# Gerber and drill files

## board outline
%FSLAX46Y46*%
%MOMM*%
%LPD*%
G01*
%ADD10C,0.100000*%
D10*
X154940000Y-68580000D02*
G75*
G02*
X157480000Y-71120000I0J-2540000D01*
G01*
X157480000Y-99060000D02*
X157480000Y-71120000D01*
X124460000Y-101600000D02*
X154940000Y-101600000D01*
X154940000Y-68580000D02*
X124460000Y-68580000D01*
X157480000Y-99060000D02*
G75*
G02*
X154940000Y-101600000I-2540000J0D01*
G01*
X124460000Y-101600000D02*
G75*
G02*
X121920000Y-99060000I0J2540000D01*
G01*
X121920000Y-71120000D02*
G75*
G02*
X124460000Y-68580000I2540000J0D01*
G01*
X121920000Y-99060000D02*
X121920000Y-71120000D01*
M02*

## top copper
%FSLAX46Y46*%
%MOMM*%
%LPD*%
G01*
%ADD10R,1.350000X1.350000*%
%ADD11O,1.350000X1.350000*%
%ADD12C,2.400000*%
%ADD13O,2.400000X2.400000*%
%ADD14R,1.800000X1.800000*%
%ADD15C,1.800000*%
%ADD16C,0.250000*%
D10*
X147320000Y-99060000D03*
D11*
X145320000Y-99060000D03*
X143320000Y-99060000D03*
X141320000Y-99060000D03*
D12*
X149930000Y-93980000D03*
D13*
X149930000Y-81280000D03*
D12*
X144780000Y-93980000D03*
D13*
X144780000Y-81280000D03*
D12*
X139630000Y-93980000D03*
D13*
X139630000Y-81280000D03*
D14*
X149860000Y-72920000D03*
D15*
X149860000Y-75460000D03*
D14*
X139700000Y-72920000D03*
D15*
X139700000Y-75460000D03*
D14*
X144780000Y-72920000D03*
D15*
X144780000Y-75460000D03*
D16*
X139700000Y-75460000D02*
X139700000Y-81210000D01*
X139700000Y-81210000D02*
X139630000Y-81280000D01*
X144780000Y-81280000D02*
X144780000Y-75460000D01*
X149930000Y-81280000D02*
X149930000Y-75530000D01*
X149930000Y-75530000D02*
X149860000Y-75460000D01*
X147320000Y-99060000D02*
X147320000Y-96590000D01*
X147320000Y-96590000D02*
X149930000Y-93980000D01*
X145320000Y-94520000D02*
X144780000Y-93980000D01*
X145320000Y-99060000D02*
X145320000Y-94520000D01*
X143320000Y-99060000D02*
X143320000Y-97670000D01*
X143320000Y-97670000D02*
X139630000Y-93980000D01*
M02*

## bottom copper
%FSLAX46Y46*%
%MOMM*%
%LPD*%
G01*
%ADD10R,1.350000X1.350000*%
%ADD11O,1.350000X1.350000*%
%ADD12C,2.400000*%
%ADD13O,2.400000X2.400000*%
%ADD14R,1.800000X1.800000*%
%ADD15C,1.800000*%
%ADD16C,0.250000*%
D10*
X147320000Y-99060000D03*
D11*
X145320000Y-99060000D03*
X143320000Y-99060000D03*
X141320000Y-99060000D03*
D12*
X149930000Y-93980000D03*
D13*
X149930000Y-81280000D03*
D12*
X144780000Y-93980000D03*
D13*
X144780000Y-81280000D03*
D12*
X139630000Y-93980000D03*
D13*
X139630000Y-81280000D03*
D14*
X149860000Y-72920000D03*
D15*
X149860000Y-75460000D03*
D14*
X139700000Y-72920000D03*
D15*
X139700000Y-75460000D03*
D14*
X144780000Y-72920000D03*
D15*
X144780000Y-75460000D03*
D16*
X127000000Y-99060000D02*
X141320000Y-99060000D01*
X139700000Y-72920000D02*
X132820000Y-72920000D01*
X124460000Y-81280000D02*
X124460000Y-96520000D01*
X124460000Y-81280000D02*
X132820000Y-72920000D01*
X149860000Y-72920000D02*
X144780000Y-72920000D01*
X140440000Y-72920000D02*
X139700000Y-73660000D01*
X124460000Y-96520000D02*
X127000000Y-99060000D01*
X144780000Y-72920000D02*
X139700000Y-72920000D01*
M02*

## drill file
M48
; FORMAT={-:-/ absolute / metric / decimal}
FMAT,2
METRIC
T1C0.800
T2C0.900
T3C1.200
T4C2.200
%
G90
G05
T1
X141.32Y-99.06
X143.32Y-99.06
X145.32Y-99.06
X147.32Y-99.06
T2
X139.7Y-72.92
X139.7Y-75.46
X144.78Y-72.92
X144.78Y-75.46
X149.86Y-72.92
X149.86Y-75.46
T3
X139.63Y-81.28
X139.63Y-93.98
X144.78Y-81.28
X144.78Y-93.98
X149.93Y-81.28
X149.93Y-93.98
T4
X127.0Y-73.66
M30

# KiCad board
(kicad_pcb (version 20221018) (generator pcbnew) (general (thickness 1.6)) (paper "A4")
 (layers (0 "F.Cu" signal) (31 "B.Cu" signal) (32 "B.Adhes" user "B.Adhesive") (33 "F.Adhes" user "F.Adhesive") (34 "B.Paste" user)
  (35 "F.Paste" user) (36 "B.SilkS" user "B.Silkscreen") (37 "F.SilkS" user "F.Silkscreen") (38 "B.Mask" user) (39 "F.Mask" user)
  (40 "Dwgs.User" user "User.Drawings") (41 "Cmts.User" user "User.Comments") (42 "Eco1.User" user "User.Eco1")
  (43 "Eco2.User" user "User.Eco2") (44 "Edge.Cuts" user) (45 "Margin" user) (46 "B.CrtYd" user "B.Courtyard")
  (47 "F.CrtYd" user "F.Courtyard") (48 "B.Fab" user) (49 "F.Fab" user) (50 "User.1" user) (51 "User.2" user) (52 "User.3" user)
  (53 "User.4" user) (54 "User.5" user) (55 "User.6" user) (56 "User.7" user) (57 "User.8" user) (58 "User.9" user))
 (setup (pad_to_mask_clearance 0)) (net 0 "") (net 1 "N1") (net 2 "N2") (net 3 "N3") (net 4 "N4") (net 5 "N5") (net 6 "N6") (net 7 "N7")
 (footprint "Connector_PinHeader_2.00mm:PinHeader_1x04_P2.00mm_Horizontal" (layer "F.Cu") (at 147.32 99.06 -90)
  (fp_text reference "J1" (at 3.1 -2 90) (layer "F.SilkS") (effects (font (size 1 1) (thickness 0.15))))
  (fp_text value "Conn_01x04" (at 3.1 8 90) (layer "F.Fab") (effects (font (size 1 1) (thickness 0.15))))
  (pad "1" thru_hole rect (at 0 0 270) (size 1.35 1.35) (drill 0.8) (layers "*.Cu" "*.Mask") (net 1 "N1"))
  (pad "2" thru_hole oval (at 0 2 270) (size 1.35 1.35) (drill 0.8) (layers "*.Cu" "*.Mask") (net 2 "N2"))
  (pad "3" thru_hole oval (at 0 4 270) (size 1.35 1.35) (drill 0.8) (layers "*.Cu" "*.Mask") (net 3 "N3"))
  (pad "4" thru_hole oval (at 0 6 270) (size 1.35 1.35) (drill 0.8) (layers "*.Cu" "*.Mask") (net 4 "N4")))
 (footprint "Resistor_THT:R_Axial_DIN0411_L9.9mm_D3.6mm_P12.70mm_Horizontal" (layer "F.Cu") (at 149.93 93.98 90)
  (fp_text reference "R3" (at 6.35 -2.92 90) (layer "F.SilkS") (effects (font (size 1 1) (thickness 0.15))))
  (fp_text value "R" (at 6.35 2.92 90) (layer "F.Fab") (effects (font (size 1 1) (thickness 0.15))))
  (pad "1" thru_hole circle (at 0 0 90) (size 2.4 2.4) (drill 1.2) (layers "*.Cu" "*.Mask") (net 1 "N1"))
  (pad "2" thru_hole oval (at 12.7 0 90) (size 2.4 2.4) (drill 1.2) (layers "*.Cu" "*.Mask") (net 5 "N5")))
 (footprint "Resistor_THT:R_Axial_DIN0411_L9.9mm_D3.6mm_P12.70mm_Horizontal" (layer "F.Cu") (at 144.78 93.98 90)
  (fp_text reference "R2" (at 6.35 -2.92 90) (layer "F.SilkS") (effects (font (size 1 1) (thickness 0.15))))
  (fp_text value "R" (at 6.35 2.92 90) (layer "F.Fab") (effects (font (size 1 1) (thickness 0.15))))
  (pad "1" thru_hole circle (at 0 0 90) (size 2.4 2.4) (drill 1.2) (layers "*.Cu" "*.Mask") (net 2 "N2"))
  (pad "2" thru_hole oval (at 12.7 0 90) (size 2.4 2.4) (drill 1.2) (layers "*.Cu" "*.Mask") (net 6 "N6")))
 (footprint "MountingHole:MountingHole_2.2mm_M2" (layer "F.Cu") (at 127 73.66)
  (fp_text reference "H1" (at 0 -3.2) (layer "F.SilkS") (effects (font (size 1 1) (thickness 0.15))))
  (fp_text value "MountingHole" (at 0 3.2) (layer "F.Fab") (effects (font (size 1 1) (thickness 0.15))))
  (pad "" np_thru_hole circle (at 0 0) (size 2.2 2.2) (drill 2.2) (layers "*.Cu" "*.Mask")))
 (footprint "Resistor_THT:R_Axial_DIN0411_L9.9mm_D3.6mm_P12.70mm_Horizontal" (layer "F.Cu") (at 139.63 93.98 90)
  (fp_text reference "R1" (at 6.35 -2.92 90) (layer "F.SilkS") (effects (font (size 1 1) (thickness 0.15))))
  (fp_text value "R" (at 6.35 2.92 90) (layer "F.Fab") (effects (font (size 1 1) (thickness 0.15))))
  (pad "1" thru_hole circle (at 0 0 90) (size 2.4 2.4) (drill 1.2) (layers "*.Cu" "*.Mask") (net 3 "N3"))
  (pad "2" thru_hole oval (at 12.7 0 90) (size 2.4 2.4) (drill 1.2) (layers "*.Cu" "*.Mask") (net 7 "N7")))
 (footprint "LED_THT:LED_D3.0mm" (layer "F.Cu") (at 149.86 72.92 -90)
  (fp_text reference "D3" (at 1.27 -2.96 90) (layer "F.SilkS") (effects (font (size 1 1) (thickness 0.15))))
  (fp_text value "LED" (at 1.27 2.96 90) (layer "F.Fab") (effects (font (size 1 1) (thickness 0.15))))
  (pad "1" thru_hole rect (at 0 0 270) (size 1.8 1.8) (drill 0.9) (layers "*.Cu" "*.Mask") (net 4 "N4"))
  (pad "2" thru_hole circle (at 2.54 0 270) (size 1.8 1.8) (drill 0.9) (layers "*.Cu" "*.Mask") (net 5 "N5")))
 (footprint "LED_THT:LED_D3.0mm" (layer "F.Cu") (at 139.7 72.92 -90)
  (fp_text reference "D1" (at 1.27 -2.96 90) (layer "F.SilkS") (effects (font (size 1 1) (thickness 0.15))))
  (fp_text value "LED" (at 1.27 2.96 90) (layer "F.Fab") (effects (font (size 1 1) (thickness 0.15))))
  (pad "1" thru_hole rect (at 0 0 270) (size 1.8 1.8) (drill 0.9) (layers "*.Cu" "*.Mask") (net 4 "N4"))
  (pad "2" thru_hole circle (at 2.54 0 270) (size 1.8 1.8) (drill 0.9) (layers "*.Cu" "*.Mask") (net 7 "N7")))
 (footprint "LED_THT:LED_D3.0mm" (layer "F.Cu") (at 144.78 72.92 -90)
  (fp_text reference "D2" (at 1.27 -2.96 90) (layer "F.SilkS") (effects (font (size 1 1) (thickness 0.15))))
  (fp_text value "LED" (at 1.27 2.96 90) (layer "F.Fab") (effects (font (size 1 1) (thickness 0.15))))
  (pad "1" thru_hole rect (at 0 0 270) (size 1.8 1.8) (drill 0.9) (layers "*.Cu" "*.Mask") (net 4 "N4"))
  (pad "2" thru_hole circle (at 2.54 0 270) (size 1.8 1.8) (drill 0.9) (layers "*.Cu" "*.Mask") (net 6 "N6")))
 (gr_arc (start 154.94 68.58) (mid 156.736051 69.323949) (end 157.48 71.12) (stroke (width 0.1) (type default)) (layer "Edge.Cuts"))
 (gr_line (start 157.48 99.06) (end 157.48 71.12) (stroke (width 0.1) (type default)) (layer "Edge.Cuts"))
 (gr_line (start 124.46 101.6) (end 154.94 101.6) (stroke (width 0.1) (type default)) (layer "Edge.Cuts"))
 (gr_line (start 154.94 68.58) (end 124.46 68.58) (stroke (width 0.1) (type default)) (layer "Edge.Cuts"))
 (gr_arc (start 157.48 99.06) (mid 156.736051 100.856051) (end 154.94 101.6) (stroke (width 0.1) (type default)) (layer "Edge.Cuts"))
 (gr_arc (start 124.46 101.6) (mid 122.663949 100.856051) (end 121.92 99.06) (stroke (width 0.1) (type default)) (layer "Edge.Cuts"))
 (gr_arc (start 121.92 71.12) (mid 122.663949 69.323949) (end 124.46 68.58) (stroke (width 0.1) (type default)) (layer "Edge.Cuts"))
 (gr_line (start 121.92 99.06) (end 121.92 71.12) (stroke (width 0.1) (type default)) (layer "Edge.Cuts"))
 (segment (start 127 99.06) (end 141.32 99.06) (width 0.25) (layer "B.Cu") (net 4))
 (segment (start 139.7 72.92) (end 132.82 72.92) (width 0.25) (layer "B.Cu") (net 4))
 (segment (start 124.46 81.28) (end 124.46 96.52) (width 0.25) (layer "B.Cu") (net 4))
 (segment (start 124.46 81.28) (end 132.82 72.92) (width 0.25) (layer "B.Cu") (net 4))
 (segment (start 149.86 72.92) (end 144.78 72.92) (width 0.25) (layer "B.Cu") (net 4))
 (segment (start 140.44 72.92) (end 139.7 73.66) (width 0.25) (layer "B.Cu") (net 4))
 (segment (start 124.46 96.52) (end 127 99.06) (width 0.25) (layer "B.Cu") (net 4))
 (segment (start 144.78 72.92) (end 139.7 72.92) (width 0.25) (layer "B.Cu") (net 4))
 (segment (start 139.7 75.46) (end 139.7 81.21) (width 0.25) (layer "F.Cu") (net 7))
 (segment (start 139.7 81.21) (end 139.63 81.28) (width 0.25) (layer "F.Cu") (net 7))
 (segment (start 144.78 81.28) (end 144.78 75.46) (width 0.25) (layer "F.Cu") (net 6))
 (segment (start 149.93 81.28) (end 149.93 75.53) (width 0.25) (layer "F.Cu") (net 5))
 (segment (start 149.93 75.53) (end 149.86 75.46) (width 0.25) (layer "F.Cu") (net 5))
 (segment (start 147.32 99.06) (end 147.32 96.59) (width 0.25) (layer "F.Cu") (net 1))
 (segment (start 147.32 96.59) (end 149.93 93.98) (width 0.25) (layer "F.Cu") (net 1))
 (segment (start 145.32 94.52) (end 144.78 93.98) (width 0.25) (layer "F.Cu") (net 2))
 (segment (start 145.32 99.06) (end 145.32 94.52) (width 0.25) (layer "F.Cu") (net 2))
 (segment (start 143.32 99.06) (end 143.32 97.67) (width 0.25) (layer "F.Cu") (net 3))
 (segment (start 143.32 97.67) (end 139.63 93.98) (width 0.25) (layer "F.Cu") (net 3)))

